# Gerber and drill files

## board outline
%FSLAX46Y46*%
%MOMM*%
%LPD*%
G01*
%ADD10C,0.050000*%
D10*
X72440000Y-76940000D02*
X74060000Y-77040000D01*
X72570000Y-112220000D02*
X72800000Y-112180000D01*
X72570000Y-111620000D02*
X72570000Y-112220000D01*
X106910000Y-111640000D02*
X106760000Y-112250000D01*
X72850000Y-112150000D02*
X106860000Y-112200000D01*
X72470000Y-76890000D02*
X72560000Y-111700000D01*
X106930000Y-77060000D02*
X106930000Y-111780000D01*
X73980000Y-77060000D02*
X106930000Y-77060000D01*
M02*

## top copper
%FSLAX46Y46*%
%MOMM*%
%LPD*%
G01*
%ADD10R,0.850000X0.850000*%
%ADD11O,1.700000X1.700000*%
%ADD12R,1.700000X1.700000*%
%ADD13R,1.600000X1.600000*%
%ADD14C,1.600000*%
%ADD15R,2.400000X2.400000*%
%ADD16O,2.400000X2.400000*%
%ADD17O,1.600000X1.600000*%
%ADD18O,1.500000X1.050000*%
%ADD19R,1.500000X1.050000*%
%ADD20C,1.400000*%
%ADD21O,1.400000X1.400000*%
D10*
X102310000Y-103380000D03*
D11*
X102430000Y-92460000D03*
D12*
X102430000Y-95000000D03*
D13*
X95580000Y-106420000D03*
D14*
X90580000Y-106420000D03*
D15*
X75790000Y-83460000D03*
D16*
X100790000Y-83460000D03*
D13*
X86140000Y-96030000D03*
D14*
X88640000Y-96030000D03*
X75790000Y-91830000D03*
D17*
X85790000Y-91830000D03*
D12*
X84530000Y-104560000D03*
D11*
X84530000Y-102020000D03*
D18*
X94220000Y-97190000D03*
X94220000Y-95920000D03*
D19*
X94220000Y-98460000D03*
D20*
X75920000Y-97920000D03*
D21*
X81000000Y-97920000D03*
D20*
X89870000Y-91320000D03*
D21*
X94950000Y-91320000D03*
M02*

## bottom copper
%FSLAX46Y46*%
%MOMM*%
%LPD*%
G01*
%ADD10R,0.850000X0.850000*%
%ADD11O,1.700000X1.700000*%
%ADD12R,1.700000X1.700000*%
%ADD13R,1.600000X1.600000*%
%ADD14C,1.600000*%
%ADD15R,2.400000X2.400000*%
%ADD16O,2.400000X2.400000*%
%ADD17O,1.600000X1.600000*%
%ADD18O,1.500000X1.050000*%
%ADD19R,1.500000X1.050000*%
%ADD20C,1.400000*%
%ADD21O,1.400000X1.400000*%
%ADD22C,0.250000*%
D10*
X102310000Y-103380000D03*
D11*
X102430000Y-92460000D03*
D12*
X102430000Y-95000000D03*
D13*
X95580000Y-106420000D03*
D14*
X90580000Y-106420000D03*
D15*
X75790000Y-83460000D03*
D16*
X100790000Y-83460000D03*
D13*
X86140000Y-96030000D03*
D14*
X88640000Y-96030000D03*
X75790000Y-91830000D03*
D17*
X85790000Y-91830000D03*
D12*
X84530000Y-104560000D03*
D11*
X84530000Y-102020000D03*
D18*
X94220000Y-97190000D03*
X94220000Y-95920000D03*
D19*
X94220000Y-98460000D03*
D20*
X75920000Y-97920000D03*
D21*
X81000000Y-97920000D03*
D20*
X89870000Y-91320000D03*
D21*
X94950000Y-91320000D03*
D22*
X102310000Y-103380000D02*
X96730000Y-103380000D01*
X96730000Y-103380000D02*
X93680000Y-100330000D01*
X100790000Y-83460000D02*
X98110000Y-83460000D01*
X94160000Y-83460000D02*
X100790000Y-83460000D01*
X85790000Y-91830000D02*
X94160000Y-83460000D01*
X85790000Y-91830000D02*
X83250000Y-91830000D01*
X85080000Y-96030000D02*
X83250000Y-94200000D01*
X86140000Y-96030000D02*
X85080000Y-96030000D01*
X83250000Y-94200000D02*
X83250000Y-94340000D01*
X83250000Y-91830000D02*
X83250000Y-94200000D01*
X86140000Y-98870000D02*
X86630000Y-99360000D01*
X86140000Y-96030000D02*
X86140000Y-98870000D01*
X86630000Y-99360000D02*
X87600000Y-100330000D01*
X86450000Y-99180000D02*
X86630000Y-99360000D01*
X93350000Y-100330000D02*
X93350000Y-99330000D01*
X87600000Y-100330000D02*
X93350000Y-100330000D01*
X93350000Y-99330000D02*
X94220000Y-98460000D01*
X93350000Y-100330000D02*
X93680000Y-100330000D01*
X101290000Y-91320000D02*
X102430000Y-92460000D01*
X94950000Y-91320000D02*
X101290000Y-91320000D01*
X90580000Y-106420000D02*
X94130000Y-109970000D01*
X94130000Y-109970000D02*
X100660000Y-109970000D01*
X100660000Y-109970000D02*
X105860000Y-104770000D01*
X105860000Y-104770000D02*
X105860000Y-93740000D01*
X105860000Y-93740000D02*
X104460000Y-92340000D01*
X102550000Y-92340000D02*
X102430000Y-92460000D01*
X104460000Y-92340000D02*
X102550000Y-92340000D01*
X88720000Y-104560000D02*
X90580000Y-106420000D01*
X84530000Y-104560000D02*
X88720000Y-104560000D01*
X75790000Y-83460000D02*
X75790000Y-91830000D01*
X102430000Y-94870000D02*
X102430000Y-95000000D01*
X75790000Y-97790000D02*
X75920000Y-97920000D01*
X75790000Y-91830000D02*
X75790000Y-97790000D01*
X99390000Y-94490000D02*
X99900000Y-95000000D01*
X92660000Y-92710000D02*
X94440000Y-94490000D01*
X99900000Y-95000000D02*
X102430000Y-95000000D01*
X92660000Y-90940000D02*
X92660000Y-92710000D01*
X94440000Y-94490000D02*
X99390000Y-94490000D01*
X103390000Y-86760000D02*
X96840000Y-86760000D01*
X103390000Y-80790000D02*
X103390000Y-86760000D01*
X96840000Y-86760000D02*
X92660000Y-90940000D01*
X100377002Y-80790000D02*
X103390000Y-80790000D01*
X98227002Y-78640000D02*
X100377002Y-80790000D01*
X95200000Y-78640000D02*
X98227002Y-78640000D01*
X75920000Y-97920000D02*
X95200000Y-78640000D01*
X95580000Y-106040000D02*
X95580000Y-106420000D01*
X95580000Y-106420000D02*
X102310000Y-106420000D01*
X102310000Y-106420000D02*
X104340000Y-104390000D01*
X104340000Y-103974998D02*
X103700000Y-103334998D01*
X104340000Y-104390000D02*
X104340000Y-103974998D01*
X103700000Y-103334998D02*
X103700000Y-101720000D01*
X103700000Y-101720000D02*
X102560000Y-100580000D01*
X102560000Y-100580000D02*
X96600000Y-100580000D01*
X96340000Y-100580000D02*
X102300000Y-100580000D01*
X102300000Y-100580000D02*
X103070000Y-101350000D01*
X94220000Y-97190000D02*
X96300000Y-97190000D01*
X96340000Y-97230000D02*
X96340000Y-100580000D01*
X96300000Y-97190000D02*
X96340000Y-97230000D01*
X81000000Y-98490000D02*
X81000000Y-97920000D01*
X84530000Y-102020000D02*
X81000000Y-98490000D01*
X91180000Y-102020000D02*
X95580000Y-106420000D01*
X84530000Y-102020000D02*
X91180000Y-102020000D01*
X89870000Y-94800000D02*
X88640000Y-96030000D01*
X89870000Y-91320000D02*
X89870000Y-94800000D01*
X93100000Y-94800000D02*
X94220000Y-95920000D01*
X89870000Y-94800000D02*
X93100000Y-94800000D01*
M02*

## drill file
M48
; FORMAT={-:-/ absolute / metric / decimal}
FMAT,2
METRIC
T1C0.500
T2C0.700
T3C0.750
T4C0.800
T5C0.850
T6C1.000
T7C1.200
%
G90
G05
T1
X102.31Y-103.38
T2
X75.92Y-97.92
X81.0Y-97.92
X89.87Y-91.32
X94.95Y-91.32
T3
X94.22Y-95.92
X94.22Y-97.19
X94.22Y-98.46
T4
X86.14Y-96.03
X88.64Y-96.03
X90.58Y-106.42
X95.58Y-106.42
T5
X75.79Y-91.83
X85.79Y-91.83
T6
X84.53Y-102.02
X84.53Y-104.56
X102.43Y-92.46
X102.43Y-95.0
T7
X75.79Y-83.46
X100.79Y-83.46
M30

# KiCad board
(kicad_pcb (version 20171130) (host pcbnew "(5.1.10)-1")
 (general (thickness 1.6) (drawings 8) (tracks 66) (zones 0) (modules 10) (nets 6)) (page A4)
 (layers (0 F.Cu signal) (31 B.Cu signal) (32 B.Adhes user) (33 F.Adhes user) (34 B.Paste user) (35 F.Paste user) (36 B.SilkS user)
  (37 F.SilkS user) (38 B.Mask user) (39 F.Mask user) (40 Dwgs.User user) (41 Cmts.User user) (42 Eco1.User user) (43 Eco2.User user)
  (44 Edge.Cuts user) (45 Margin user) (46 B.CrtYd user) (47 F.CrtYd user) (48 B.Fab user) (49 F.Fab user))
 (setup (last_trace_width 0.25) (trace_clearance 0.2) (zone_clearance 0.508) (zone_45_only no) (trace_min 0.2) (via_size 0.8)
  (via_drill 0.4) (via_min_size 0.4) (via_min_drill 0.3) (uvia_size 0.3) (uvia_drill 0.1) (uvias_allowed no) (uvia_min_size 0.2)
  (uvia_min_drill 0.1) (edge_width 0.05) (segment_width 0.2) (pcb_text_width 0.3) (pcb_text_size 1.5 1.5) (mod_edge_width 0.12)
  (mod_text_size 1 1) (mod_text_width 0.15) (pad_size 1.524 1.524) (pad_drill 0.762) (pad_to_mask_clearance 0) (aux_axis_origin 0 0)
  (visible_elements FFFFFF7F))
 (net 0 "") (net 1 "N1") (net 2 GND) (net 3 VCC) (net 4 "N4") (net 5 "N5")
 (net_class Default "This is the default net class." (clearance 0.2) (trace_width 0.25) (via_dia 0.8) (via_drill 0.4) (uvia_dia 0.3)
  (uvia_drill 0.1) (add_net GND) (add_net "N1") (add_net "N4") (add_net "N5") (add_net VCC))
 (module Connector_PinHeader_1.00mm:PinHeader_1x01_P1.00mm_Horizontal (layer F.Cu) (at 102.31 103.38)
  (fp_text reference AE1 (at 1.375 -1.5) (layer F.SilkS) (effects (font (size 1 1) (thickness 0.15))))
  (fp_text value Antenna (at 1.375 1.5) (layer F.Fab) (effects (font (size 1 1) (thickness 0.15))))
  (pad 1 thru_hole rect (at 0 0) (size 0.85 0.85) (drill 0.5) (layers *.Cu *.Mask) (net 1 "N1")))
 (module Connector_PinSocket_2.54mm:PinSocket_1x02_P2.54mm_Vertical (layer F.Cu) (at 102.43 95 180)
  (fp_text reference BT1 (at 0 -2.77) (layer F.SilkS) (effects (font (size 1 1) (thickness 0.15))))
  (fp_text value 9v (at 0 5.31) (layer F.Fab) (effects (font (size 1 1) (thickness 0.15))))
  (pad 2 thru_hole oval (at 0 2.54 180) (size 1.7 1.7) (drill 1) (layers *.Cu *.Mask) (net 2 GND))
  (pad 1 thru_hole rect (at 0 0 180) (size 1.7 1.7) (drill 1) (layers *.Cu *.Mask) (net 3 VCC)))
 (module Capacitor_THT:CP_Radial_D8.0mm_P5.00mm (layer F.Cu) (at 95.58 106.42 180)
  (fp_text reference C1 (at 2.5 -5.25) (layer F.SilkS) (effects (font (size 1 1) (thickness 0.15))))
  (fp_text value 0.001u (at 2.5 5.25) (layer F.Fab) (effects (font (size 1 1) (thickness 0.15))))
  (pad 1 thru_hole rect (at 0 0 180) (size 1.6 1.6) (drill 0.8) (layers *.Cu *.Mask) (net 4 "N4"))
  (pad 2 thru_hole circle (at 5 0 180) (size 1.6 1.6) (drill 0.8) (layers *.Cu *.Mask) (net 2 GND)))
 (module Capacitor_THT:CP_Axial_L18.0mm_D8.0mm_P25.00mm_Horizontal (layer F.Cu) (at 75.79 83.46)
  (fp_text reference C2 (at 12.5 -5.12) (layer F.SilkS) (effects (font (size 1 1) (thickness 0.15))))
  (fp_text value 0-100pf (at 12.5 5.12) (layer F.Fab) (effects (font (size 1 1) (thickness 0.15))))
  (pad 1 thru_hole rect (at 0 0) (size 2.4 2.4) (drill 1.2) (layers *.Cu *.Mask) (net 3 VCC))
  (pad 2 thru_hole oval (at 25 0) (size 2.4 2.4) (drill 1.2) (layers *.Cu *.Mask) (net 1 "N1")))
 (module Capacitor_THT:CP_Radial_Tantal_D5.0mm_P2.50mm (layer F.Cu) (at 86.14 96.03)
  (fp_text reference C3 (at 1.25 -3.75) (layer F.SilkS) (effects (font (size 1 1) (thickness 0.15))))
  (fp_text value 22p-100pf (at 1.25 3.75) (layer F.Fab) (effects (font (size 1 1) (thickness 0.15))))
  (pad 1 thru_hole rect (at 0 0) (size 1.6 1.6) (drill 0.8) (layers *.Cu *.Mask) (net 1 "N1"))
  (pad 2 thru_hole circle (at 2.5 0) (size 1.6 1.6) (drill 0.8) (layers *.Cu *.Mask) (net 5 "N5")))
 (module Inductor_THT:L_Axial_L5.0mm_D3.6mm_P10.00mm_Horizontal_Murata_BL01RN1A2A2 (layer F.Cu) (at 75.79 91.83)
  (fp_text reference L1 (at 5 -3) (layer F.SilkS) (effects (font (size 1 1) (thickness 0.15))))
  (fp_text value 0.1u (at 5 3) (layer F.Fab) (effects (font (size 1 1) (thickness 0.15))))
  (pad 1 thru_hole circle (at 0 0) (size 1.6 1.6) (drill 0.85) (layers *.Cu *.Mask) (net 3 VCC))
  (pad 2 thru_hole oval (at 10 0) (size 1.6 1.6) (drill 0.85) (layers *.Cu *.Mask) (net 1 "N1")))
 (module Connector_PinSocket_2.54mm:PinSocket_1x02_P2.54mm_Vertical (layer F.Cu) (at 84.53 104.56 180)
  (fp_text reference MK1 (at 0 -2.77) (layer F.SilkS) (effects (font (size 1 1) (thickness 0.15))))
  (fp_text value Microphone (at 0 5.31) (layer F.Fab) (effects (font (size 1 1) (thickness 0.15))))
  (pad 1 thru_hole rect (at 0 0 180) (size 1.7 1.7) (drill 1) (layers *.Cu *.Mask) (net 2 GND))
  (pad 2 thru_hole oval (at 0 2.54 180) (size 1.7 1.7) (drill 1) (layers *.Cu *.Mask) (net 4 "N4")))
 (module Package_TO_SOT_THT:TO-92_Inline (layer F.Cu) (at 94.22 98.46 90)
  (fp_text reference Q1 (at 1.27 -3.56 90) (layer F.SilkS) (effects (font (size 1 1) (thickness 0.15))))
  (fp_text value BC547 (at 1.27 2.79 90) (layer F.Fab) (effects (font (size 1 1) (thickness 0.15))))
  (pad 2 thru_hole oval (at 1.27 0 90) (size 1.05 1.5) (drill 0.75) (layers *.Cu *.Mask) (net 4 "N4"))
  (pad 3 thru_hole oval (at 2.54 0 90) (size 1.05 1.5) (drill 0.75) (layers *.Cu *.Mask) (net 5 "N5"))
  (pad 1 thru_hole rect (at 0 0 90) (size 1.05 1.5) (drill 0.75) (layers *.Cu *.Mask) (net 1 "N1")))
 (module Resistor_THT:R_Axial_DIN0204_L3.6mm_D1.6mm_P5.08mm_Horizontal (layer F.Cu) (at 75.92 97.92)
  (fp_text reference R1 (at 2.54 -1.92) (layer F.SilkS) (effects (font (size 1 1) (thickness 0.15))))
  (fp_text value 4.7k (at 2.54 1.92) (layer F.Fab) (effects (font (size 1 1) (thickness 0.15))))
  (pad 1 thru_hole circle (at 0 0) (size 1.4 1.4) (drill 0.7) (layers *.Cu *.Mask) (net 3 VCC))
  (pad 2 thru_hole oval (at 5.08 0) (size 1.4 1.4) (drill 0.7) (layers *.Cu *.Mask) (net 4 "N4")))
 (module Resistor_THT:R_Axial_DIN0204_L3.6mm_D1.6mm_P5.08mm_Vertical (layer F.Cu) (at 89.87 91.32)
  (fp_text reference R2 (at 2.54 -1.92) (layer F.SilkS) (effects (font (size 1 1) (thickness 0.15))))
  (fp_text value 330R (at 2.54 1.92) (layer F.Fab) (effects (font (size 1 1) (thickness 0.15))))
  (pad 1 thru_hole circle (at 0 0) (size 1.4 1.4) (drill 0.7) (layers *.Cu *.Mask) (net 5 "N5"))
  (pad 2 thru_hole oval (at 5.08 0) (size 1.4 1.4) (drill 0.7) (layers *.Cu *.Mask) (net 2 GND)))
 (gr_line (start 72.44 76.94) (end 74.06 77.04) (layer Edge.Cuts) (width 0.05))
 (gr_line (start 72.57 112.22) (end 72.8 112.18) (layer Edge.Cuts) (width 0.05))
 (gr_line (start 72.57 111.62) (end 72.57 112.22) (layer Edge.Cuts) (width 0.05))
 (gr_line (start 106.91 111.64) (end 106.76 112.25) (layer Edge.Cuts) (width 0.05))
 (gr_line (start 72.85 112.15) (end 106.86 112.2) (layer Edge.Cuts) (width 0.05))
 (gr_line (start 72.47 76.89) (end 72.56 111.7) (layer Edge.Cuts) (width 0.05))
 (gr_line (start 106.93 77.06) (end 106.93 111.78) (layer Edge.Cuts) (width 0.05))
 (gr_line (start 73.98 77.06) (end 106.93 77.06) (layer Edge.Cuts) (width 0.05))
 (segment (start 102.31 103.38) (end 96.73 103.38) (width 0.25) (layer B.Cu) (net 1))
 (segment (start 96.73 103.38) (end 93.68 100.33) (width 0.25) (layer B.Cu) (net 1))
 (segment (start 100.79 83.46) (end 98.11 83.46) (width 0.25) (layer B.Cu) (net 1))
 (segment (start 94.16 83.46) (end 100.79 83.46) (width 0.25) (layer B.Cu) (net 1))
 (segment (start 85.79 91.83) (end 94.16 83.46) (width 0.25) (layer B.Cu) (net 1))
 (segment (start 85.79 91.83) (end 83.25 91.83) (width 0.25) (layer B.Cu) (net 1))
 (segment (start 85.08 96.03) (end 83.25 94.2) (width 0.25) (layer B.Cu) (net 1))
 (segment (start 86.14 96.03) (end 85.08 96.03) (width 0.25) (layer B.Cu) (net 1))
 (segment (start 83.25 94.2) (end 83.25 94.34) (width 0.25) (layer B.Cu) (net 1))
 (segment (start 83.25 91.83) (end 83.25 94.2) (width 0.25) (layer B.Cu) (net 1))
 (segment (start 86.14 98.87) (end 86.63 99.36) (width 0.25) (layer B.Cu) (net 1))
 (segment (start 86.14 96.03) (end 86.14 98.87) (width 0.25) (layer B.Cu) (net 1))
 (segment (start 86.63 99.36) (end 87.6 100.33) (width 0.25) (layer B.Cu) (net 1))
 (segment (start 86.45 99.18) (end 86.63 99.36) (width 0.25) (layer B.Cu) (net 1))
 (segment (start 93.35 100.33) (end 93.35 99.33) (width 0.25) (layer B.Cu) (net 1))
 (segment (start 87.6 100.33) (end 93.35 100.33) (width 0.25) (layer B.Cu) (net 1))
 (segment (start 93.35 99.33) (end 94.22 98.46) (width 0.25) (layer B.Cu) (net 1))
 (segment (start 93.35 100.33) (end 93.68 100.33) (width 0.25) (layer B.Cu) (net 1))
 (segment (start 101.29 91.32) (end 102.43 92.46) (width 0.25) (layer B.Cu) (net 2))
 (segment (start 94.95 91.32) (end 101.29 91.32) (width 0.25) (layer B.Cu) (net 2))
 (segment (start 90.58 106.42) (end 94.13 109.97) (width 0.25) (layer B.Cu) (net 2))
 (segment (start 94.13 109.97) (end 100.66 109.97) (width 0.25) (layer B.Cu) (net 2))
 (segment (start 100.66 109.97) (end 105.86 104.77) (width 0.25) (layer B.Cu) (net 2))
 (segment (start 105.86 104.77) (end 105.86 93.74) (width 0.25) (layer B.Cu) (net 2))
 (segment (start 105.86 93.74) (end 104.46 92.34) (width 0.25) (layer B.Cu) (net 2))
 (segment (start 102.55 92.34) (end 102.43 92.46) (width 0.25) (layer B.Cu) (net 2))
 (segment (start 104.46 92.34) (end 102.55 92.34) (width 0.25) (layer B.Cu) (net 2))
 (segment (start 88.72 104.56) (end 90.58 106.42) (width 0.25) (layer B.Cu) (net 2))
 (segment (start 84.53 104.56) (end 88.72 104.56) (width 0.25) (layer B.Cu) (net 2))
 (segment (start 75.79 83.46) (end 75.79 91.83) (width 0.25) (layer B.Cu) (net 3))
 (segment (start 102.43 94.87) (end 102.43 95) (width 0.25) (layer B.Cu) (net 3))
 (segment (start 75.79 97.79) (end 75.92 97.92) (width 0.25) (layer B.Cu) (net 3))
 (segment (start 75.79 91.83) (end 75.79 97.79) (width 0.25) (layer B.Cu) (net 3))
 (segment (start 99.39 94.49) (end 99.9 95) (width 0.25) (layer B.Cu) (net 3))
 (segment (start 92.66 92.71) (end 94.44 94.49) (width 0.25) (layer B.Cu) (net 3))
 (segment (start 99.9 95) (end 102.43 95) (width 0.25) (layer B.Cu) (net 3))
 (segment (start 92.66 90.94) (end 92.66 92.71) (width 0.25) (layer B.Cu) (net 3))
 (segment (start 94.44 94.49) (end 99.39 94.49) (width 0.25) (layer B.Cu) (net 3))
 (segment (start 103.39 86.76) (end 96.84 86.76) (width 0.25) (layer B.Cu) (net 3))
 (segment (start 103.39 80.79) (end 103.39 86.76) (width 0.25) (layer B.Cu) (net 3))
 (segment (start 96.84 86.76) (end 92.66 90.94) (width 0.25) (layer B.Cu) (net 3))
 (segment (start 100.377002 80.79) (end 103.39 80.79) (width 0.25) (layer B.Cu) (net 3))
 (segment (start 98.227002 78.64) (end 100.377002 80.79) (width 0.25) (layer B.Cu) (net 3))
 (segment (start 95.2 78.64) (end 98.227002 78.64) (width 0.25) (layer B.Cu) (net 3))
 (segment (start 75.92 97.92) (end 95.2 78.64) (width 0.25) (layer B.Cu) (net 3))
 (segment (start 95.58 106.04) (end 95.58 106.42) (width 0.25) (layer B.Cu) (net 4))
 (segment (start 95.58 106.42) (end 102.31 106.42) (width 0.25) (layer B.Cu) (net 4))
 (segment (start 102.31 106.42) (end 104.34 104.39) (width 0.25) (layer B.Cu) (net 4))
 (segment (start 104.34 103.974998) (end 103.7 103.334998) (width 0.25) (layer B.Cu) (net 4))
 (segment (start 104.34 104.39) (end 104.34 103.974998) (width 0.25) (layer B.Cu) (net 4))
 (segment (start 103.7 103.334998) (end 103.7 101.72) (width 0.25) (layer B.Cu) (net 4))
 (segment (start 103.7 101.72) (end 102.56 100.58) (width 0.25) (layer B.Cu) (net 4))
 (segment (start 102.56 100.58) (end 96.6 100.58) (width 0.25) (layer B.Cu) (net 4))
 (segment (start 96.34 100.58) (end 102.3 100.58) (width 0.25) (layer B.Cu) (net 4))
 (segment (start 102.3 100.58) (end 103.07 101.35) (width 0.25) (layer B.Cu) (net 4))
 (segment (start 94.22 97.19) (end 96.3 97.19) (width 0.25) (layer B.Cu) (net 4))
 (segment (start 96.34 97.23) (end 96.34 100.58) (width 0.25) (layer B.Cu) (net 4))
 (segment (start 96.3 97.19) (end 96.34 97.23) (width 0.25) (layer B.Cu) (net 4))
 (segment (start 81 98.49) (end 81 97.92) (width 0.25) (layer B.Cu) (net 4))
 (segment (start 84.53 102.02) (end 81 98.49) (width 0.25) (layer B.Cu) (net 4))
 (segment (start 91.18 102.02) (end 95.58 106.42) (width 0.25) (layer B.Cu) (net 4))
 (segment (start 84.53 102.02) (end 91.18 102.02) (width 0.25) (layer B.Cu) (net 4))
 (segment (start 89.87 94.8) (end 88.64 96.03) (width 0.25) (layer B.Cu) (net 5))
 (segment (start 89.87 91.32) (end 89.87 94.8) (width 0.25) (layer B.Cu) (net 5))
 (segment (start 93.1 94.8) (end 94.22 95.92) (width 0.25) (layer B.Cu) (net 5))
 (segment (start 89.87 94.8) (end 93.1 94.8) (width 0.25) (layer B.Cu) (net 5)))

